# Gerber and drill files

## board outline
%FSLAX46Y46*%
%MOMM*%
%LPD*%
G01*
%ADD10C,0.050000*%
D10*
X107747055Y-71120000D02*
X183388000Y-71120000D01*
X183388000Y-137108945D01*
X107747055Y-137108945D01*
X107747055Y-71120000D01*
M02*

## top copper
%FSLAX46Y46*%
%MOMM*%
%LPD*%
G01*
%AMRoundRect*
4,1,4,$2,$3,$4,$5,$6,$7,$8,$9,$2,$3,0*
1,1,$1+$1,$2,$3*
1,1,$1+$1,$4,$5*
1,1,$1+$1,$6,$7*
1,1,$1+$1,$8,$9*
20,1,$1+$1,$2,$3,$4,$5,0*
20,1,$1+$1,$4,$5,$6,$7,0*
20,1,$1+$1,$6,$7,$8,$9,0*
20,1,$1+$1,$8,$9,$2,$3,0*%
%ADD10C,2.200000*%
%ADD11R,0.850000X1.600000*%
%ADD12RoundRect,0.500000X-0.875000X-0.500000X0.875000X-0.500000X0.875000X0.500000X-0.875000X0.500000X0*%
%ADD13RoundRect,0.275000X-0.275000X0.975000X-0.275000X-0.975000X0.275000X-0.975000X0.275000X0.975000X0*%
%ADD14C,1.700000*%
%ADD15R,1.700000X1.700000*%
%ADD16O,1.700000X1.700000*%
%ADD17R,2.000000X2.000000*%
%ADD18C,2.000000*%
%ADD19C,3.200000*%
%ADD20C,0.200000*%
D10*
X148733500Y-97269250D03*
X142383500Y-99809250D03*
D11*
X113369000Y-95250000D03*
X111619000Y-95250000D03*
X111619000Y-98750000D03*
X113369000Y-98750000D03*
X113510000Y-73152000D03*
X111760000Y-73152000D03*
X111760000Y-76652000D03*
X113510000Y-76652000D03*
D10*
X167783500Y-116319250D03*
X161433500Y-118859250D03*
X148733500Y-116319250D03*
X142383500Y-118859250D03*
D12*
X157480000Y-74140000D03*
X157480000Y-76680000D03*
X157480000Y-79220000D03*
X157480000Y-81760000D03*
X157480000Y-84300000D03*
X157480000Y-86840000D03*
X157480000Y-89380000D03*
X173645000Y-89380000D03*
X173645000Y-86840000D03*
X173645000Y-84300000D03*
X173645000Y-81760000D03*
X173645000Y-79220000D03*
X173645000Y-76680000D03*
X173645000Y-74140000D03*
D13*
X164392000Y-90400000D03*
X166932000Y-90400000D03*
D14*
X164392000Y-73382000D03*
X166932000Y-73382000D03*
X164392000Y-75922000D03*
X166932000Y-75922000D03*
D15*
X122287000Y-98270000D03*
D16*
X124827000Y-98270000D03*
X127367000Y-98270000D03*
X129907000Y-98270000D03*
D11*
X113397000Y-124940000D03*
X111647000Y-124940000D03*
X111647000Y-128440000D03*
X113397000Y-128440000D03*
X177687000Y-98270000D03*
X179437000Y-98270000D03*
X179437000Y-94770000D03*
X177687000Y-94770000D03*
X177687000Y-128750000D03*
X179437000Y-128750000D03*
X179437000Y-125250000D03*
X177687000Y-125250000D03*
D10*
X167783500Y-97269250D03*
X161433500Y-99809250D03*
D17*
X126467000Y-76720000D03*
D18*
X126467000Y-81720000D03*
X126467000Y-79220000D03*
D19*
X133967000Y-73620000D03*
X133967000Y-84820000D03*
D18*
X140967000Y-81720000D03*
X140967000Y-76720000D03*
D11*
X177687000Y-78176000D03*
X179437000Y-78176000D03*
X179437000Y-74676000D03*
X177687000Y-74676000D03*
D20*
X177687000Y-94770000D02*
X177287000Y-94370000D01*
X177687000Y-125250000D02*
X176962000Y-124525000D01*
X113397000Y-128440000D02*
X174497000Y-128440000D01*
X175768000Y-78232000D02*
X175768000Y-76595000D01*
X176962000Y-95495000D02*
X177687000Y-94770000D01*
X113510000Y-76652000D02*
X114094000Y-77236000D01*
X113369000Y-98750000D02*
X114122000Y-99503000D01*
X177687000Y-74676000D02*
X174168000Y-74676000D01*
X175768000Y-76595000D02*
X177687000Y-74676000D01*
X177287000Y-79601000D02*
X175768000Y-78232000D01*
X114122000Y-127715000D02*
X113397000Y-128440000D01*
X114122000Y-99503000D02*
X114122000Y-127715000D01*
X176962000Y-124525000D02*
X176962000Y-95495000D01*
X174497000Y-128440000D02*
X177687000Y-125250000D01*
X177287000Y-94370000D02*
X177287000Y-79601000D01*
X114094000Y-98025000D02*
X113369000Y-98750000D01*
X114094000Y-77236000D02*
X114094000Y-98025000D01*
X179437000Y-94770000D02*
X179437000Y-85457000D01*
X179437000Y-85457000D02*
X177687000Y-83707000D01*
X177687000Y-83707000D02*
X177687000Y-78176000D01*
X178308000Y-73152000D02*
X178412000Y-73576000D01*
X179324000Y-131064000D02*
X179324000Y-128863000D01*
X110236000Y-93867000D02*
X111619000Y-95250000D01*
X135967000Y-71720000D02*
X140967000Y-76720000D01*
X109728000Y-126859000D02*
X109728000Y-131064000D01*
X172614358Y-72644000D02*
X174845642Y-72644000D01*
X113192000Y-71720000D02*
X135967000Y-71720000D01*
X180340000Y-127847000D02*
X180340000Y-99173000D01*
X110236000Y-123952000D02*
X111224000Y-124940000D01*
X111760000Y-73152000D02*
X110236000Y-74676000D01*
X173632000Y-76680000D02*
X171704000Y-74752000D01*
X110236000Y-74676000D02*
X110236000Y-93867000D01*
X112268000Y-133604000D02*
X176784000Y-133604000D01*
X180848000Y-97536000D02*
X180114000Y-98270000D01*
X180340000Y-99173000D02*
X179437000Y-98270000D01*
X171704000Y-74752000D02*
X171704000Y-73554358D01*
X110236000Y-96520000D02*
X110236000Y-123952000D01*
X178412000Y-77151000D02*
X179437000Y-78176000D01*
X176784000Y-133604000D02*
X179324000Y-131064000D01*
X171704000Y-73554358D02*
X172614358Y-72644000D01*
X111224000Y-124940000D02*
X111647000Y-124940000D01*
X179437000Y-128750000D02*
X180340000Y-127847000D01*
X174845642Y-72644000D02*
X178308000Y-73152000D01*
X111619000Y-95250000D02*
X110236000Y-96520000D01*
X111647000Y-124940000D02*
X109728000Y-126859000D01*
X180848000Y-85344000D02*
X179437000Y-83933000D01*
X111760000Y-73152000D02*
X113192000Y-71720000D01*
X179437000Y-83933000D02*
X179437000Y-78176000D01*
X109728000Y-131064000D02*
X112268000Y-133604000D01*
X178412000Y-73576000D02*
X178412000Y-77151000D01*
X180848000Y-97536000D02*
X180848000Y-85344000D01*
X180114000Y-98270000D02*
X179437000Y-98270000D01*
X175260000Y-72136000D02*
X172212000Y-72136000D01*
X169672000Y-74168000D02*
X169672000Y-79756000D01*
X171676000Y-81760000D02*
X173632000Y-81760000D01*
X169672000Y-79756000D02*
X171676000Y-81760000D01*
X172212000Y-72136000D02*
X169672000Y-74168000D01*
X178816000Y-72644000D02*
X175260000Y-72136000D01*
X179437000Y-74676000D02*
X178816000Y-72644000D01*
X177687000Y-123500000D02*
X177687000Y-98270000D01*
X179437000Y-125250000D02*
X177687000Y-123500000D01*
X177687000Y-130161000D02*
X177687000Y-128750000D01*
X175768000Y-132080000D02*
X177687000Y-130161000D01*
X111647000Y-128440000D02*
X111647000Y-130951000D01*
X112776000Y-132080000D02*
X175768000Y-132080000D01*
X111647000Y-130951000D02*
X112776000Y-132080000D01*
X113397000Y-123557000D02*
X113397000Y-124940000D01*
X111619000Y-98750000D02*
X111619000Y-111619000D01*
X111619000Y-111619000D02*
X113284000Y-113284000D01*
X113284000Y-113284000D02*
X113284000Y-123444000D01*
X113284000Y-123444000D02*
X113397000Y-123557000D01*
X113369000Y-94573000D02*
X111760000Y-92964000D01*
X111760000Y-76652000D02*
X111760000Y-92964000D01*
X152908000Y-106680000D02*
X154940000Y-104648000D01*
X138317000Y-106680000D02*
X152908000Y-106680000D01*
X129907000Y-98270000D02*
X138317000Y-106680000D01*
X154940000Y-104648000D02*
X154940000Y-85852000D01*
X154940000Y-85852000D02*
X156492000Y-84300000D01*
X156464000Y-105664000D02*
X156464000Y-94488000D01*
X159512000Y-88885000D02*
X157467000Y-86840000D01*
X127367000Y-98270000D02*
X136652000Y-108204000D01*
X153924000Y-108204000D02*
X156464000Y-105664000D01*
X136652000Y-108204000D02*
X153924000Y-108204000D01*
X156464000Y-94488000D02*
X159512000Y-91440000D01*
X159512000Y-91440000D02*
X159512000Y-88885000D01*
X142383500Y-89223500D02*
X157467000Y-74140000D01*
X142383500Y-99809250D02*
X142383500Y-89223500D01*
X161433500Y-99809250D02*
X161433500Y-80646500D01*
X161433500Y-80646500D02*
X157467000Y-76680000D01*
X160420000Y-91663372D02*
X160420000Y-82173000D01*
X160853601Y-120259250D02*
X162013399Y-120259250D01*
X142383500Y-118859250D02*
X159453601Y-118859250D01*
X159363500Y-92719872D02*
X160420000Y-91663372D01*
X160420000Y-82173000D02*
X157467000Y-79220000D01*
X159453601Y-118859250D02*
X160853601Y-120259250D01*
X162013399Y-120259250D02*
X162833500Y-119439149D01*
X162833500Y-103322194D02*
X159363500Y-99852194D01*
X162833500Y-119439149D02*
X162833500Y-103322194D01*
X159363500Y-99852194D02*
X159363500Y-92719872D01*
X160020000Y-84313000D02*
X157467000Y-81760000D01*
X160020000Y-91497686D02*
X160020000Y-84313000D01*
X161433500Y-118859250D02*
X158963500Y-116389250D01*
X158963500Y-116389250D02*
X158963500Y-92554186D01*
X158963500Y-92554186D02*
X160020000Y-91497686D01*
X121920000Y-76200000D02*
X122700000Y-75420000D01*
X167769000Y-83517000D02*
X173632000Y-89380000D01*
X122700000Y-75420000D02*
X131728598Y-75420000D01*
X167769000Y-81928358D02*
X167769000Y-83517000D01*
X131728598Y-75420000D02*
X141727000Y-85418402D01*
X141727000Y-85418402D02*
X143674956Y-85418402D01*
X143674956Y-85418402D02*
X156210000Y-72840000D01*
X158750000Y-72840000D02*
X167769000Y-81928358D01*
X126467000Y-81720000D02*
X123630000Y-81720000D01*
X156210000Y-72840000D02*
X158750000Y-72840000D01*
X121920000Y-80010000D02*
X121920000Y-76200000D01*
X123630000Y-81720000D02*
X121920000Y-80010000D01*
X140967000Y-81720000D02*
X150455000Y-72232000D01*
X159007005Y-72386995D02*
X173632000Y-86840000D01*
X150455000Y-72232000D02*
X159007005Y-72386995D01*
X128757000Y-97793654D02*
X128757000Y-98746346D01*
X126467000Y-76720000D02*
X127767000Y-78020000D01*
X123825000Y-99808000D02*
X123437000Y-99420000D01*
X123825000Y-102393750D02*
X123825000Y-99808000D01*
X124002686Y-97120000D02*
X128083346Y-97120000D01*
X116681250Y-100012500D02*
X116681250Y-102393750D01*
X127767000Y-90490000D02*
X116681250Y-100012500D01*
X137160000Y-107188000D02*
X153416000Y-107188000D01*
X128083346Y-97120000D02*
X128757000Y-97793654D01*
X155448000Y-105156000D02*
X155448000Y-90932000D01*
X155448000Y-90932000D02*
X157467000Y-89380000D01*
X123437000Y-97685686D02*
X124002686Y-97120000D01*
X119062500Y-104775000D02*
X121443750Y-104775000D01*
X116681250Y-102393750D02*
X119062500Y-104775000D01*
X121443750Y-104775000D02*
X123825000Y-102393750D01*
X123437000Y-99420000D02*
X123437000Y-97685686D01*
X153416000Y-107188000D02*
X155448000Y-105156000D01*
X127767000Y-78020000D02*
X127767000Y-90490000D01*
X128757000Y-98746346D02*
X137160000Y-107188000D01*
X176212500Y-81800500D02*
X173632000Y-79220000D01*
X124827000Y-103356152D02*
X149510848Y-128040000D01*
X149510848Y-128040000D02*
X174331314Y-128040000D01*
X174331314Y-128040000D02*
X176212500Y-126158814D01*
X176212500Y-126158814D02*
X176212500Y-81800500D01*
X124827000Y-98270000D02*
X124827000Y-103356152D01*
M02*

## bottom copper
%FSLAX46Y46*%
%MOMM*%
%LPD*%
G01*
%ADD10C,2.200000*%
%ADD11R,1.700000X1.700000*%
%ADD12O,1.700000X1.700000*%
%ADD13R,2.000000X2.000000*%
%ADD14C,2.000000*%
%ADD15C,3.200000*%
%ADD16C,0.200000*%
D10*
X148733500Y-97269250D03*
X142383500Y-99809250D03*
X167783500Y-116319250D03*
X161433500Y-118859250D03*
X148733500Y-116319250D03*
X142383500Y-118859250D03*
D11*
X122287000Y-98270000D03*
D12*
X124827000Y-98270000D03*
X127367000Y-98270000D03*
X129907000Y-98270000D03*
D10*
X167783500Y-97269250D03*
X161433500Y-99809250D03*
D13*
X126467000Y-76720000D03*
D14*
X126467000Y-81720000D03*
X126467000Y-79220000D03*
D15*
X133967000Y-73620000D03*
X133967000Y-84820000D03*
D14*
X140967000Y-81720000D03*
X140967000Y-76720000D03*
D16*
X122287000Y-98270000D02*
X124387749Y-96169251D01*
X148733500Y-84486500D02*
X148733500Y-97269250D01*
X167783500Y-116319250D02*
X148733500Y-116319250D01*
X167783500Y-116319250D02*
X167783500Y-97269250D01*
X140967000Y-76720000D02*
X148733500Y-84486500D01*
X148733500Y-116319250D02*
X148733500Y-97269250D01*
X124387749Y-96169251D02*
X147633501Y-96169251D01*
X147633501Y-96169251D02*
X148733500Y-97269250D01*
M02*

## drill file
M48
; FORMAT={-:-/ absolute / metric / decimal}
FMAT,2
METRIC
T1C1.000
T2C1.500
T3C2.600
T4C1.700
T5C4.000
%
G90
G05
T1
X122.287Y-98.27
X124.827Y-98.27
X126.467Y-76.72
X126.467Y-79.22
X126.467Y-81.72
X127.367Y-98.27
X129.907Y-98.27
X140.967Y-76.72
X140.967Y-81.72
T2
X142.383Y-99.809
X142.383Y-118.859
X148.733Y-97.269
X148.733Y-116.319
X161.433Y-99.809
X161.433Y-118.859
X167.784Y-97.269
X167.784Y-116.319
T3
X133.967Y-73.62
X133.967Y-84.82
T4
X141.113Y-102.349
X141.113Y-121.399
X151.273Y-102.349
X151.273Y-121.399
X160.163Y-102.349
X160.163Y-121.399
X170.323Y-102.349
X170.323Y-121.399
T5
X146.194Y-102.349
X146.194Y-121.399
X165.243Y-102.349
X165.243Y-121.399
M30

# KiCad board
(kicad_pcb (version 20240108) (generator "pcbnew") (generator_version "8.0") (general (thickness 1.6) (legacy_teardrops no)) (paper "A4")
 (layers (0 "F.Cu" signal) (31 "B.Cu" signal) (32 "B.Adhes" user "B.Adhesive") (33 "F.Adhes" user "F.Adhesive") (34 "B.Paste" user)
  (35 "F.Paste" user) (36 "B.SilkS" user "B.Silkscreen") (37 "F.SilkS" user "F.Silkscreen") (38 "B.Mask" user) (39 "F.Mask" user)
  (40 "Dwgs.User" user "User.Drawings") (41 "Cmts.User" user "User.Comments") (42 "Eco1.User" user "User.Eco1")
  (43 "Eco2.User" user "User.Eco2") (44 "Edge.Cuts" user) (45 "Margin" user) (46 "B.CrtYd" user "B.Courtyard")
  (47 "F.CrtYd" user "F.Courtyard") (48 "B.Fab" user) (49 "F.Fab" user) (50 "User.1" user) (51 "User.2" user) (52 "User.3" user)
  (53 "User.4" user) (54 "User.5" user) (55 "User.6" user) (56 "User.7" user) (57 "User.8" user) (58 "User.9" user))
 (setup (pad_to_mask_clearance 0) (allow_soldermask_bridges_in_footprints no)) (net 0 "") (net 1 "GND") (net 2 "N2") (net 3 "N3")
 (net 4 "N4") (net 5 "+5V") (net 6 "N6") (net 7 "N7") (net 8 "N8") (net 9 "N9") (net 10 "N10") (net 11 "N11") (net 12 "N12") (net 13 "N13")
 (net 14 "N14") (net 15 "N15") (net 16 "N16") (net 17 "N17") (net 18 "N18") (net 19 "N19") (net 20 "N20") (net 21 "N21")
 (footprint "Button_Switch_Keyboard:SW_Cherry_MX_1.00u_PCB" (layer "F.Cu") (at 148.7335 97.26925)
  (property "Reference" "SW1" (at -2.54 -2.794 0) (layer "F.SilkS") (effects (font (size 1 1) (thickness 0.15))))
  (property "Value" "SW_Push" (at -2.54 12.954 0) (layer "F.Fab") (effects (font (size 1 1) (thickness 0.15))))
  (pad "" np_thru_hole circle (at -7.62 5.08) (size 1.7 1.7) (drill 1.7) (layers "*.Cu" "*.Mask"))
  (pad "" np_thru_hole circle (at -2.54 5.08) (size 4 4) (drill 4) (layers "*.Cu" "*.Mask"))
  (pad "" np_thru_hole circle (at 2.54 5.08) (size 1.7 1.7) (drill 1.7) (layers "*.Cu" "*.Mask"))
  (pad "1" thru_hole circle (at 0 0) (size 2.2 2.2) (drill 1.5) (layers "*.Cu" "*.Mask") (remove_unused_layers no) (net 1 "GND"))
  (pad "2" thru_hole circle (at -6.35 2.54) (size 2.2 2.2) (drill 1.5) (layers "*.Cu" "*.Mask") (remove_unused_layers no) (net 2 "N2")))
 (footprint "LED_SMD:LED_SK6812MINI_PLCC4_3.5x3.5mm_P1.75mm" (layer "F.Cu") (at 112.494 97 -90)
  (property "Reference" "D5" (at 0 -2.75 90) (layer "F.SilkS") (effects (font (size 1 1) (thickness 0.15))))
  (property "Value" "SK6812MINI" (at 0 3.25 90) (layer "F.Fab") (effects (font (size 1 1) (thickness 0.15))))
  (pad "1" smd rect (at -1.75 -0.875 270) (size 1.6 0.85) (layers "F.Cu" "F.Paste" "F.Mask") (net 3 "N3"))
  (pad "2" smd rect (at -1.75 0.875 270) (size 1.6 0.85) (layers "F.Cu" "F.Paste" "F.Mask") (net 1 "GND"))
  (pad "3" smd rect (at 1.75 0.875 270) (size 1.6 0.85) (layers "F.Cu" "F.Paste" "F.Mask") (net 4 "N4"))
  (pad "4" smd rect (at 1.75 -0.875 270) (size 1.6 0.85) (layers "F.Cu" "F.Paste" "F.Mask") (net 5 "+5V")))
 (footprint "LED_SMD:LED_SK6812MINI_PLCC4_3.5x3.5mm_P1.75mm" (layer "F.Cu") (at 112.635 74.902 -90)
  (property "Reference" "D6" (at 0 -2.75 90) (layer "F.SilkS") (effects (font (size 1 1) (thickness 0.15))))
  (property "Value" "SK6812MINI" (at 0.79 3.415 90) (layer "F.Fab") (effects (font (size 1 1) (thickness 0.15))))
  (pad "1" smd rect (at -1.75 -0.875 270) (size 1.6 0.85) (layers "F.Cu" "F.Paste" "F.Mask") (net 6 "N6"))
  (pad "2" smd rect (at -1.75 0.875 270) (size 1.6 0.85) (layers "F.Cu" "F.Paste" "F.Mask") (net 1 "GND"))
  (pad "3" smd rect (at 1.75 0.875 270) (size 1.6 0.85) (layers "F.Cu" "F.Paste" "F.Mask") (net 3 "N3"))
  (pad "4" smd rect (at 1.75 -0.875 270) (size 1.6 0.85) (layers "F.Cu" "F.Paste" "F.Mask") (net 5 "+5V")))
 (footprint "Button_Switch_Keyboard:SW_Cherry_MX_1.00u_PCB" (layer "F.Cu") (at 167.7835 116.31925)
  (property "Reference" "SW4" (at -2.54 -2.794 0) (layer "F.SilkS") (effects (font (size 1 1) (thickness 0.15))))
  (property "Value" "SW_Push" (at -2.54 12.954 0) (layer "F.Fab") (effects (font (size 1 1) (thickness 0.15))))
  (pad "" np_thru_hole circle (at -7.62 5.08) (size 1.7 1.7) (drill 1.7) (layers "*.Cu" "*.Mask"))
  (pad "" np_thru_hole circle (at -2.54 5.08) (size 4 4) (drill 4) (layers "F&B.Cu" "*.Mask"))
  (pad "" np_thru_hole circle (at 2.54 5.08) (size 1.7 1.7) (drill 1.7) (layers "*.Cu" "*.Mask"))
  (pad "1" thru_hole circle (at 0 0) (size 2.2 2.2) (drill 1.5) (layers "*.Cu" "*.Mask") (remove_unused_layers no) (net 1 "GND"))
  (pad "2" thru_hole circle (at -6.35 2.54) (size 2.2 2.2) (drill 1.5) (layers "*.Cu" "*.Mask") (remove_unused_layers no) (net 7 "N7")))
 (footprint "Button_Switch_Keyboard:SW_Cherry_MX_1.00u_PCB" (layer "F.Cu") (at 148.7335 116.31925)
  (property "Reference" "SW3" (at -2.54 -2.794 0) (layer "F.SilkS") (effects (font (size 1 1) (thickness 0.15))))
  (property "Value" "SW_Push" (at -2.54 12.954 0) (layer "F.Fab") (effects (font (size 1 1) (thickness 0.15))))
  (pad "" np_thru_hole circle (at -7.62 5.08) (size 1.7 1.7) (drill 1.7) (layers "*.Cu" "*.Mask"))
  (pad "" np_thru_hole circle (at -2.54 5.08) (size 4 4) (drill 4) (layers "F&B.Cu" "*.Mask"))
  (pad "" np_thru_hole circle (at 2.54 5.08) (size 1.7 1.7) (drill 1.7) (layers "*.Cu" "*.Mask"))
  (pad "1" thru_hole circle (at 0 0) (size 2.2 2.2) (drill 1.5) (layers "*.Cu" "*.Mask") (remove_unused_layers no) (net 1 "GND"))
  (pad "2" thru_hole circle (at -6.35 2.54) (size 2.2 2.2) (drill 1.5) (layers "*.Cu" "*.Mask") (remove_unused_layers no) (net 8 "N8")))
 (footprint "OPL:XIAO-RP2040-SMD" (layer "F.Cu") (at 165.48 81.76)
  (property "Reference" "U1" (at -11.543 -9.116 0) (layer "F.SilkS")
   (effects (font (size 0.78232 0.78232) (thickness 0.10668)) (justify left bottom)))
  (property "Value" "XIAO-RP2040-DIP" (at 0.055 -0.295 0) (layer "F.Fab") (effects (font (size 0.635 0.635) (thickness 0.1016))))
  (pad "1" smd roundrect (at -8 -7.62) (size 2.75 2) (layers "F.Cu" "F.Paste" "F.Mask") (roundrect_rratio 0.25) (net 2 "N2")
   (solder_mask_margin 0.0508) (thermal_bridge_angle 45))
  (pad "2" smd roundrect (at -8 -5.08) (size 2.75 2) (layers "F.Cu" "F.Paste" "F.Mask") (roundrect_rratio 0.25) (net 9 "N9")
   (solder_mask_margin 0.0508) (thermal_bridge_angle 45))
  (pad "3" smd roundrect (at -8 -2.54) (size 2.75 2) (layers "F.Cu" "F.Paste" "F.Mask") (roundrect_rratio 0.25) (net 8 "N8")
   (solder_mask_margin 0.0508) (thermal_bridge_angle 45))
  (pad "4" smd roundrect (at -8 0) (size 2.75 2) (layers "F.Cu" "F.Paste" "F.Mask") (roundrect_rratio 0.25) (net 7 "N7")
   (solder_mask_margin 0.0508) (thermal_bridge_angle 45))
  (pad "5" smd roundrect (at -8 2.54) (size 2.75 2) (layers "F.Cu" "F.Paste" "F.Mask") (roundrect_rratio 0.25) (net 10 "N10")
   (solder_mask_margin 0.0508) (thermal_bridge_angle 45))
  (pad "6" smd roundrect (at -8 5.08) (size 2.75 2) (layers "F.Cu" "F.Paste" "F.Mask") (roundrect_rratio 0.25) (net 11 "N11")
   (solder_mask_margin 0.0508) (thermal_bridge_angle 45))
  (pad "7" smd roundrect (at -8 7.62) (size 2.75 2) (layers "F.Cu" "F.Paste" "F.Mask") (roundrect_rratio 0.25) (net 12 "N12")
   (solder_mask_margin 0.0508) (thermal_bridge_angle 45))
  (pad "8" smd roundrect (at 8.165 7.62) (size 2.75 2) (layers "F.Cu" "F.Paste" "F.Mask") (roundrect_rratio 0.25) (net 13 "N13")
   (solder_mask_margin 0.0508) (thermal_bridge_angle 45))
  (pad "9" smd roundrect (at 8.165 5.08) (size 2.75 2) (layers "F.Cu" "F.Paste" "F.Mask") (roundrect_rratio 0.25) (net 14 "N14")
   (solder_mask_margin 0.0508) (thermal_bridge_angle 45))
  (pad "10" smd roundrect (at 8.165 2.54) (size 2.75 2) (layers "F.Cu" "F.Paste" "F.Mask") (roundrect_rratio 0.25) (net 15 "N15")
   (solder_mask_margin 0.0508) (thermal_bridge_angle 45))
  (pad "11" smd roundrect (at 8.165 0) (size 2.75 2) (layers "F.Cu" "F.Paste" "F.Mask") (roundrect_rratio 0.25) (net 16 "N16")
   (solder_mask_margin 0.0508) (thermal_bridge_angle 45))
  (pad "12" smd roundrect (at 8.165 -2.54) (size 2.75 2) (layers "F.Cu" "F.Paste" "F.Mask") (roundrect_rratio 0.25) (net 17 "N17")
   (solder_mask_margin 0.0508) (thermal_bridge_angle 45))
  (pad "13" smd roundrect (at 8.165 -5.08) (size 2.75 2) (layers "F.Cu" "F.Paste" "F.Mask") (roundrect_rratio 0.25) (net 1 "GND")
   (solder_mask_margin 0.0508) (thermal_bridge_angle 45))
  (pad "14" smd roundrect (at 8.165 -7.62) (size 2.75 2) (layers "F.Cu" "F.Paste" "F.Mask") (roundrect_rratio 0.25) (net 5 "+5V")
   (solder_mask_margin 0.0508) (thermal_bridge_angle 45))
  (pad "15" smd roundrect (at -1.088 8.64 270) (size 2.5 1.1) (layers "F.Cu" "F.Paste" "F.Mask") (roundrect_rratio 0.25)
   (thermal_bridge_angle 45))
  (pad "16" smd roundrect (at 1.452 8.64 270) (size 2.5 1.1) (layers "F.Cu" "F.Paste" "F.Mask") (roundrect_rratio 0.25)
   (thermal_bridge_angle 45))
  (pad "17" smd circle (at -1.088 -8.378) (size 1.7 1.7) (layers "F.Cu" "F.Paste" "F.Mask"))
  (pad "18" smd circle (at 1.452 -8.378) (size 1.7 1.7) (layers "F.Cu" "F.Paste" "F.Mask"))
  (pad "19" smd circle (at -1.088 -5.838) (size 1.7 1.7) (layers "F.Cu" "F.Paste" "F.Mask"))
  (pad "20" smd circle (at 1.452 -5.838) (size 1.7 1.7) (layers "F.Cu" "F.Paste" "F.Mask")))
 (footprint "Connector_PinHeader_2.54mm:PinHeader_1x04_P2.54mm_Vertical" (layer "F.Cu") (at 122.287 98.27 90)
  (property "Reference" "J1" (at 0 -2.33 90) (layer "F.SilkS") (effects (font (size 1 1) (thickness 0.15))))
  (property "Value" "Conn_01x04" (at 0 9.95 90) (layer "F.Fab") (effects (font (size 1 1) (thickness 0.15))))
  (pad "1" thru_hole rect (at 0 0 90) (size 1.7 1.7) (drill 1) (layers "*.Cu" "*.Mask") (remove_unused_layers no) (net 1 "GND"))
  (pad "2" thru_hole oval (at 0 2.54 90) (size 1.7 1.7) (drill 1) (layers "*.Cu" "*.Mask") (remove_unused_layers no) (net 17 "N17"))
  (pad "3" thru_hole oval (at 0 5.08 90) (size 1.7 1.7) (drill 1) (layers "*.Cu" "*.Mask") (remove_unused_layers no) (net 11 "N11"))
  (pad "4" thru_hole oval (at 0 7.62 90) (size 1.7 1.7) (drill 1) (layers "*.Cu" "*.Mask") (remove_unused_layers no) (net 10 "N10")))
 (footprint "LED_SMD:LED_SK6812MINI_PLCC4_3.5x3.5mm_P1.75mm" (layer "F.Cu") (at 112.522 126.69 -90)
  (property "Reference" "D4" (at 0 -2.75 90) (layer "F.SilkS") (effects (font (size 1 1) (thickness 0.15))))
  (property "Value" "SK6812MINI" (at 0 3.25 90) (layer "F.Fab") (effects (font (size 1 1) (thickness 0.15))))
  (pad "1" smd rect (at -1.75 -0.875 270) (size 1.6 0.85) (layers "F.Cu" "F.Paste" "F.Mask") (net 4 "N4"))
  (pad "2" smd rect (at -1.75 0.875 270) (size 1.6 0.85) (layers "F.Cu" "F.Paste" "F.Mask") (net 1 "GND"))
  (pad "3" smd rect (at 1.75 0.875 270) (size 1.6 0.85) (layers "F.Cu" "F.Paste" "F.Mask") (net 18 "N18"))
  (pad "4" smd rect (at 1.75 -0.875 270) (size 1.6 0.85) (layers "F.Cu" "F.Paste" "F.Mask") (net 5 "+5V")))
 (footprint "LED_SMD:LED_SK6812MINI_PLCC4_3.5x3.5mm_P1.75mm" (layer "F.Cu") (at 178.562 96.52 90)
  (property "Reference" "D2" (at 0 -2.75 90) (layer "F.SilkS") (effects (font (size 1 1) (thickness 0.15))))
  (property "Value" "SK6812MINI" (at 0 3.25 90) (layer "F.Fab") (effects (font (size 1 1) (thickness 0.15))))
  (pad "1" smd rect (at -1.75 -0.875 90) (size 1.6 0.85) (layers "F.Cu" "F.Paste" "F.Mask") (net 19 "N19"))
  (pad "2" smd rect (at -1.75 0.875 90) (size 1.6 0.85) (layers "F.Cu" "F.Paste" "F.Mask") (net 1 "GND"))
  (pad "3" smd rect (at 1.75 0.875 90) (size 1.6 0.85) (layers "F.Cu" "F.Paste" "F.Mask") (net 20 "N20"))
  (pad "4" smd rect (at 1.75 -0.875 90) (size 1.6 0.85) (layers "F.Cu" "F.Paste" "F.Mask") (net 5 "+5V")))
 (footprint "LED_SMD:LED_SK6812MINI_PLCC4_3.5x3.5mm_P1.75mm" (layer "F.Cu") (at 178.562 127 90)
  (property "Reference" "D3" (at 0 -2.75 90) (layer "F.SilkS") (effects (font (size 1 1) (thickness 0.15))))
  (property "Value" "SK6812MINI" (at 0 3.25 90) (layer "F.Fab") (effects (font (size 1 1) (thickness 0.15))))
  (pad "1" smd rect (at -1.75 -0.875 90) (size 1.6 0.85) (layers "F.Cu" "F.Paste" "F.Mask") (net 18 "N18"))
  (pad "2" smd rect (at -1.75 0.875 90) (size 1.6 0.85) (layers "F.Cu" "F.Paste" "F.Mask") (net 1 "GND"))
  (pad "3" smd rect (at 1.75 0.875 90) (size 1.6 0.85) (layers "F.Cu" "F.Paste" "F.Mask") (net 19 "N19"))
  (pad "4" smd rect (at 1.75 -0.875 90) (size 1.6 0.85) (layers "F.Cu" "F.Paste" "F.Mask") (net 5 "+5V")))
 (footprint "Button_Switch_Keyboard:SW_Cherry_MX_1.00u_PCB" (layer "F.Cu") (at 167.7835 97.26925)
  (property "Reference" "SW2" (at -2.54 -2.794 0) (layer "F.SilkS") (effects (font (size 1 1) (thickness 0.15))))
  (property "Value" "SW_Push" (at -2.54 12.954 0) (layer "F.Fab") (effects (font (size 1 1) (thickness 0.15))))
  (pad "" np_thru_hole circle (at -7.62 5.08) (size 1.7 1.7) (drill 1.7) (layers "*.Cu" "*.Mask"))
  (pad "" np_thru_hole circle (at -2.54 5.08) (size 4 4) (drill 4) (layers "F&B.Cu" "*.Mask"))
  (pad "" np_thru_hole circle (at 2.54 5.08) (size 1.7 1.7) (drill 1.7) (layers "*.Cu" "*.Mask"))
  (pad "1" thru_hole circle (at 0 0) (size 2.2 2.2) (drill 1.5) (layers "*.Cu" "*.Mask") (remove_unused_layers no) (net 1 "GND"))
  (pad "2" thru_hole circle (at -6.35 2.54) (size 2.2 2.2) (drill 1.5) (layers "*.Cu" "*.Mask") (remove_unused_layers no) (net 9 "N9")))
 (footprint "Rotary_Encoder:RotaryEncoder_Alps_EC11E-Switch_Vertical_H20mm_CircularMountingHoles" (layer "F.Cu") (at 126.467 76.72)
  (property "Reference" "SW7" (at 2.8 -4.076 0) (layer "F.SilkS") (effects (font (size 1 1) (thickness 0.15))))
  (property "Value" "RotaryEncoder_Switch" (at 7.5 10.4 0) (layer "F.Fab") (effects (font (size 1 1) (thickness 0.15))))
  (pad "A" thru_hole rect (at 0 0) (size 2 2) (drill 1) (layers "*.Cu" "*.Mask") (remove_unused_layers no) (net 12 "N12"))
  (pad "B" thru_hole circle (at 0 5) (size 2 2) (drill 1) (layers "*.Cu" "*.Mask") (remove_unused_layers no) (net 13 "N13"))
  (pad "C" thru_hole circle (at 0 2.5) (size 2 2) (drill 1) (layers "*.Cu" "*.Mask") (remove_unused_layers no) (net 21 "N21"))
  (pad "MP" thru_hole circle (at 7.5 -3.1) (size 3.2 3.2) (drill 2.6) (layers "*.Cu" "*.Mask") (remove_unused_layers no))
  (pad "MP" thru_hole circle (at 7.5 8.1) (size 3.2 3.2) (drill 2.6) (layers "*.Cu" "*.Mask") (remove_unused_layers no))
  (pad "S1" thru_hole circle (at 14.5 5) (size 2 2) (drill 1) (layers "*.Cu" "*.Mask") (remove_unused_layers no) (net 14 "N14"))
  (pad "S2" thru_hole circle (at 14.5 0) (size 2 2) (drill 1) (layers "*.Cu" "*.Mask") (remove_unused_layers no) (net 1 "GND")))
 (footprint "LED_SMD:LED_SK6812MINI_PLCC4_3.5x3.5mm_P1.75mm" (layer "F.Cu") (at 178.562 76.426 90)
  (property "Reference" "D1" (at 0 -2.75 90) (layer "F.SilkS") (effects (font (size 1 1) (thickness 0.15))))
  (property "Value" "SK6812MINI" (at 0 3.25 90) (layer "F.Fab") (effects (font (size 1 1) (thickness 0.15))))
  (pad "1" smd rect (at -1.75 -0.875 90) (size 1.6 0.85) (layers "F.Cu" "F.Paste" "F.Mask") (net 20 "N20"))
  (pad "2" smd rect (at -1.75 0.875 90) (size 1.6 0.85) (layers "F.Cu" "F.Paste" "F.Mask") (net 1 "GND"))
  (pad "3" smd rect (at 1.75 0.875 90) (size 1.6 0.85) (layers "F.Cu" "F.Paste" "F.Mask") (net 16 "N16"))
  (pad "4" smd rect (at 1.75 -0.875 90) (size 1.6 0.85) (layers "F.Cu" "F.Paste" "F.Mask") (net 5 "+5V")))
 (gr_rect (start 107.747055 71.12) (end 183.388 137.108945) (stroke (width 0.05) (type default)) (fill none) (layer "Edge.Cuts"))
 (segment (start 177.687 94.77) (end 177.287 94.37) (width 0.2) (layer "F.Cu") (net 5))
 (segment (start 177.687 125.25) (end 176.962 124.525) (width 0.2) (layer "F.Cu") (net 5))
 (segment (start 113.397 128.44) (end 174.497 128.44) (width 0.2) (layer "F.Cu") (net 5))
 (segment (start 175.768 78.232) (end 175.768 76.595) (width 0.2) (layer "F.Cu") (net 5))
 (segment (start 176.962 95.495) (end 177.687 94.77) (width 0.2) (layer "F.Cu") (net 5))
 (segment (start 113.51 76.652) (end 114.094 77.236) (width 0.2) (layer "F.Cu") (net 5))
 (segment (start 113.369 98.75) (end 114.122 99.503) (width 0.2) (layer "F.Cu") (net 5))
 (segment (start 177.687 74.676) (end 174.168 74.676) (width 0.2) (layer "F.Cu") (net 5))
 (segment (start 175.768 76.595) (end 177.687 74.676) (width 0.2) (layer "F.Cu") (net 5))
 (segment (start 177.287 79.601) (end 175.768 78.232) (width 0.2) (layer "F.Cu") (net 5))
 (segment (start 114.122 127.715) (end 113.397 128.44) (width 0.2) (layer "F.Cu") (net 5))
 (segment (start 114.122 99.503) (end 114.122 127.715) (width 0.2) (layer "F.Cu") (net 5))
 (segment (start 176.962 124.525) (end 176.962 95.495) (width 0.2) (layer "F.Cu") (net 5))
 (segment (start 174.497 128.44) (end 177.687 125.25) (width 0.2) (layer "F.Cu") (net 5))
 (segment (start 177.287 94.37) (end 177.287 79.601) (width 0.2) (layer "F.Cu") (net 5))
 (segment (start 114.094 98.025) (end 113.369 98.75) (width 0.2) (layer "F.Cu") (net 5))
 (segment (start 114.094 77.236) (end 114.094 98.025) (width 0.2) (layer "F.Cu") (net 5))
 (segment (start 179.437 94.77) (end 179.437 85.457) (width 0.2) (layer "F.Cu") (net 20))
 (segment (start 179.437 85.457) (end 177.687 83.707) (width 0.2) (layer "F.Cu") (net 20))
 (segment (start 177.687 83.707) (end 177.687 78.176) (width 0.2) (layer "F.Cu") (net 20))
 (segment (start 178.308 73.152) (end 178.412 73.576) (width 0.2) (layer "F.Cu") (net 1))
 (segment (start 179.324 131.064) (end 179.324 128.863) (width 0.2) (layer "F.Cu") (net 1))
 (segment (start 110.236 93.867) (end 111.619 95.25) (width 0.2) (layer "F.Cu") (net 1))
 (segment (start 135.967 71.72) (end 140.967 76.72) (width 0.2) (layer "F.Cu") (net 1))
 (segment (start 109.728 126.859) (end 109.728 131.064) (width 0.2) (layer "F.Cu") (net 1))
 (segment (start 172.614358 72.644) (end 174.845642 72.644) (width 0.2) (layer "F.Cu") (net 1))
 (segment (start 113.192 71.72) (end 135.967 71.72) (width 0.2) (layer "F.Cu") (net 1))
 (segment (start 180.34 127.847) (end 180.34 99.173) (width 0.2) (layer "F.Cu") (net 1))
 (segment (start 110.236 123.952) (end 111.224 124.94) (width 0.2) (layer "F.Cu") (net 1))
 (segment (start 111.76 73.152) (end 110.236 74.676) (width 0.2) (layer "F.Cu") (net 1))
 (segment (start 173.632 76.68) (end 171.704 74.752) (width 0.2) (layer "F.Cu") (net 1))
 (segment (start 110.236 74.676) (end 110.236 93.867) (width 0.2) (layer "F.Cu") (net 1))
 (segment (start 112.268 133.604) (end 176.784 133.604) (width 0.2) (layer "F.Cu") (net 1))
 (segment (start 180.848 97.536) (end 180.114 98.27) (width 0.2) (layer "F.Cu") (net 1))
 (segment (start 180.34 99.173) (end 179.437 98.27) (width 0.2) (layer "F.Cu") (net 1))
 (segment (start 171.704 74.752) (end 171.704 73.554358) (width 0.2) (layer "F.Cu") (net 1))
 (segment (start 110.236 96.52) (end 110.236 123.952) (width 0.2) (layer "F.Cu") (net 1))
 (segment (start 178.412 77.151) (end 179.437 78.176) (width 0.2) (layer "F.Cu") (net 1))
 (segment (start 176.784 133.604) (end 179.324 131.064) (width 0.2) (layer "F.Cu") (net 1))
 (segment (start 171.704 73.554358) (end 172.614358 72.644) (width 0.2) (layer "F.Cu") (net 1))
 (segment (start 111.224 124.94) (end 111.647 124.94) (width 0.2) (layer "F.Cu") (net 1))
 (segment (start 179.437 128.75) (end 180.34 127.847) (width 0.2) (layer "F.Cu") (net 1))
 (segment (start 174.845642 72.644) (end 178.308 73.152) (width 0.2) (layer "F.Cu") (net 1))
 (segment (start 111.619 95.25) (end 110.236 96.52) (width 0.2) (layer "F.Cu") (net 1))
 (segment (start 111.647 124.94) (end 109.728 126.859) (width 0.2) (layer "F.Cu") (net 1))
 (segment (start 180.848 85.344) (end 179.437 83.933) (width 0.2) (layer "F.Cu") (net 1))
 (segment (start 111.76 73.152) (end 113.192 71.72) (width 0.2) (layer "F.Cu") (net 1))
 (segment (start 179.437 83.933) (end 179.437 78.176) (width 0.2) (layer "F.Cu") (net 1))
 (segment (start 109.728 131.064) (end 112.268 133.604) (width 0.2) (layer "F.Cu") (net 1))
 (segment (start 178.412 73.576) (end 178.412 77.151) (width 0.2) (layer "F.Cu") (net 1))
 (segment (start 180.848 97.536) (end 180.848 85.344) (width 0.2) (layer "F.Cu") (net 1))
 (segment (start 180.114 98.27) (end 179.437 98.27) (width 0.2) (layer "F.Cu") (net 1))
 (segment (start 122.287 98.27) (end 124.387749 96.169251) (width 0.2) (layer "B.Cu") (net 1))
 (segment (start 148.7335 84.4865) (end 148.7335 97.26925) (width 0.2) (layer "B.Cu") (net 1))
 (segment (start 167.7835 116.31925) (end 148.7335 116.31925) (width 0.2) (layer "B.Cu") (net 1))
 (segment (start 167.7835 116.31925) (end 167.7835 97.26925) (width 0.2) (layer "B.Cu") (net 1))
 (segment (start 140.967 76.72) (end 148.7335 84.4865) (width 0.2) (layer "B.Cu") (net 1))
 (segment (start 148.7335 116.31925) (end 148.7335 97.26925) (width 0.2) (layer "B.Cu") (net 1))
 (segment (start 124.387749 96.169251) (end 147.633501 96.169251) (width 0.2) (layer "B.Cu") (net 1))
 (segment (start 147.633501 96.169251) (end 148.7335 97.26925) (width 0.2) (layer "B.Cu") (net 1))
 (segment (start 175.26 72.136) (end 172.212 72.136) (width 0.2) (layer "F.Cu") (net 16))
 (segment (start 169.672 74.168) (end 169.672 79.756) (width 0.2) (layer "F.Cu") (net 16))
 (segment (start 171.676 81.76) (end 173.632 81.76) (width 0.2) (layer "F.Cu") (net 16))
 (segment (start 169.672 79.756) (end 171.676 81.76) (width 0.2) (layer "F.Cu") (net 16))
 (segment (start 172.212 72.136) (end 169.672 74.168) (width 0.2) (layer "F.Cu") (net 16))
 (segment (start 178.816 72.644) (end 175.26 72.136) (width 0.2) (layer "F.Cu") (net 16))
 (segment (start 179.437 74.676) (end 178.816 72.644) (width 0.2) (layer "F.Cu") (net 16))
 (segment (start 177.687 123.5) (end 177.687 98.27) (width 0.2) (layer "F.Cu") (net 19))
 (segment (start 179.437 125.25) (end 177.687 123.5) (width 0.2) (layer "F.Cu") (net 19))
 (segment (start 177.687 130.161) (end 177.687 128.75) (width 0.2) (layer "F.Cu") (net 18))
 (segment (start 175.768 132.08) (end 177.687 130.161) (width 0.2) (layer "F.Cu") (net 18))
 (segment (start 111.647 128.44) (end 111.647 130.951) (width 0.2) (layer "F.Cu") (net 18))
 (segment (start 112.776 132.08) (end 175.768 132.08) (width 0.2) (layer "F.Cu") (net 18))
 (segment (start 111.647 130.951) (end 112.776 132.08) (width 0.2) (layer "F.Cu") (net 18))
 (segment (start 113.397 123.557) (end 113.397 124.94) (width 0.2) (layer "F.Cu") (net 4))
 (segment (start 111.619 98.75) (end 111.619 111.619) (width 0.2) (layer "F.Cu") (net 4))
 (segment (start 111.619 111.619) (end 113.284 113.284) (width 0.2) (layer "F.Cu") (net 4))
 (segment (start 113.284 113.284) (end 113.284 123.444) (width 0.2) (layer "F.Cu") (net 4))
 (segment (start 113.284 123.444) (end 113.397 123.557) (width 0.2) (layer "F.Cu") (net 4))
 (segment (start 113.369 94.573) (end 111.76 92.964) (width 0.2) (layer "F.Cu") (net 3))
 (segment (start 111.76 76.652) (end 111.76 92.964) (width 0.2) (layer "F.Cu") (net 3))
 (segment (start 152.908 106.68) (end 154.94 104.648) (width 0.2) (layer "F.Cu") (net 10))
 (segment (start 138.317 106.68) (end 152.908 106.68) (width 0.2) (layer "F.Cu") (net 10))
 (segment (start 129.907 98.27) (end 138.317 106.68) (width 0.2) (layer "F.Cu") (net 10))
 (segment (start 154.94 104.648) (end 154.94 85.852) (width 0.2) (layer "F.Cu") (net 10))
 (segment (start 154.94 85.852) (end 156.492 84.3) (width 0.2) (layer "F.Cu") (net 10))
 (segment (start 156.464 105.664) (end 156.464 94.488) (width 0.2) (layer "F.Cu") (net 11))
 (segment (start 159.512 88.885) (end 157.467 86.84) (width 0.2) (layer "F.Cu") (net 11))
 (segment (start 127.367 98.27) (end 136.652 108.204) (width 0.2) (layer "F.Cu") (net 11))
 (segment (start 153.924 108.204) (end 156.464 105.664) (width 0.2) (layer "F.Cu") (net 11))
 (segment (start 136.652 108.204) (end 153.924 108.204) (width 0.2) (layer "F.Cu") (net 11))
 (segment (start 156.464 94.488) (end 159.512 91.44) (width 0.2) (layer "F.Cu") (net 11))
 (segment (start 159.512 91.44) (end 159.512 88.885) (width 0.2) (layer "F.Cu") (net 11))
 (segment (start 142.3835 89.2235) (end 157.467 74.14) (width 0.2) (layer "F.Cu") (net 2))
 (segment (start 142.3835 99.80925) (end 142.3835 89.2235) (width 0.2) (layer "F.Cu") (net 2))
 (segment (start 161.4335 99.80925) (end 161.4335 80.6465) (width 0.2) (layer "F.Cu") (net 9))
 (segment (start 161.4335 80.6465) (end 157.467 76.68) (width 0.2) (layer "F.Cu") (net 9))
 (segment (start 160.42 91.663372) (end 160.42 82.173) (width 0.2) (layer "F.Cu") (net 8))
 (segment (start 160.853601 120.25925) (end 162.013399 120.25925) (width 0.2) (layer "F.Cu") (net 8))
 (segment (start 142.3835 118.85925) (end 159.453601 118.85925) (width 0.2) (layer "F.Cu") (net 8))
 (segment (start 159.3635 92.719872) (end 160.42 91.663372) (width 0.2) (layer "F.Cu") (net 8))
 (segment (start 160.42 82.173) (end 157.467 79.22) (width 0.2) (layer "F.Cu") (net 8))
 (segment (start 159.453601 118.85925) (end 160.853601 120.25925) (width 0.2) (layer "F.Cu") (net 8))
 (segment (start 162.013399 120.25925) (end 162.8335 119.439149) (width 0.2) (layer "F.Cu") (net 8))
 (segment (start 162.8335 103.322194) (end 159.3635 99.852194) (width 0.2) (layer "F.Cu") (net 8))
 (segment (start 162.8335 119.439149) (end 162.8335 103.322194) (width 0.2) (layer "F.Cu") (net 8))
 (segment (start 159.3635 99.852194) (end 159.3635 92.719872) (width 0.2) (layer "F.Cu") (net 8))
 (segment (start 160.02 84.313) (end 157.467 81.76) (width 0.2) (layer "F.Cu") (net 7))
 (segment (start 160.02 91.497686) (end 160.02 84.313) (width 0.2) (layer "F.Cu") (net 7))
 (segment (start 161.4335 118.85925) (end 158.9635 116.38925) (width 0.2) (layer "F.Cu") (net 7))
 (segment (start 158.9635 116.38925) (end 158.9635 92.554186) (width 0.2) (layer "F.Cu") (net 7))
 (segment (start 158.9635 92.554186) (end 160.02 91.497686) (width 0.2) (layer "F.Cu") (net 7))
 (segment (start 121.92 76.2) (end 122.7 75.42) (width 0.2) (layer "F.Cu") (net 13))
 (segment (start 167.769 83.517) (end 173.632 89.38) (width 0.2) (layer "F.Cu") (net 13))
 (segment (start 122.7 75.42) (end 131.728598 75.42) (width 0.2) (layer "F.Cu") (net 13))
 (segment (start 167.769 81.928358) (end 167.769 83.517) (width 0.2) (layer "F.Cu") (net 13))
 (segment (start 131.728598 75.42) (end 141.727 85.418402) (width 0.2) (layer "F.Cu") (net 13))
 (segment (start 141.727 85.418402) (end 143.674956 85.418402) (width 0.2) (layer "F.Cu") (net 13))
 (segment (start 143.674956 85.418402) (end 156.21 72.84) (width 0.2) (layer "F.Cu") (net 13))
 (segment (start 158.75 72.84) (end 167.769 81.928358) (width 0.2) (layer "F.Cu") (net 13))
 (segment (start 126.467 81.72) (end 123.63 81.72) (width 0.2) (layer "F.Cu") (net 13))
 (segment (start 156.21 72.84) (end 158.75 72.84) (width 0.2) (layer "F.Cu") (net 13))
 (segment (start 121.92 80.01) (end 121.92 76.2) (width 0.2) (layer "F.Cu") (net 13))
 (segment (start 123.63 81.72) (end 121.92 80.01) (width 0.2) (layer "F.Cu") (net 13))
 (segment (start 140.967 81.72) (end 150.455 72.232) (width 0.2) (layer "F.Cu") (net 14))
 (segment (start 159.007005 72.386995) (end 173.632 86.84) (width 0.2) (layer "F.Cu") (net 14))
 (segment (start 150.455 72.232) (end 159.007005 72.386995) (width 0.2) (layer "F.Cu") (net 14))
 (segment (start 128.757 97.793654) (end 128.757 98.746346) (width 0.2) (layer "F.Cu") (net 12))
 (segment (start 126.467 76.72) (end 127.767 78.02) (width 0.2) (layer "F.Cu") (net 12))
 (segment (start 123.825 99.808) (end 123.437 99.42) (width 0.2) (layer "F.Cu") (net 12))
 (segment (start 123.825 102.39375) (end 123.825 99.808) (width 0.2) (layer "F.Cu") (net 12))
 (segment (start 124.002686 97.12) (end 128.083346 97.12) (width 0.2) (layer "F.Cu") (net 12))
 (segment (start 116.68125 100.0125) (end 116.68125 102.39375) (width 0.2) (layer "F.Cu") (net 12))
 (segment (start 127.767 90.49) (end 116.68125 100.0125) (width 0.2) (layer "F.Cu") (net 12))
 (segment (start 137.16 107.188) (end 153.416 107.188) (width 0.2) (layer "F.Cu") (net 12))
 (segment (start 128.083346 97.12) (end 128.757 97.793654) (width 0.2) (layer "F.Cu") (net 12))
 (segment (start 155.448 105.156) (end 155.448 90.932) (width 0.2) (layer "F.Cu") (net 12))
 (segment (start 155.448 90.932) (end 157.467 89.38) (width 0.2) (layer "F.Cu") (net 12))
 (segment (start 123.437 97.685686) (end 124.002686 97.12) (width 0.2) (layer "F.Cu") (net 12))
 (segment (start 119.0625 104.775) (end 121.44375 104.775) (width 0.2) (layer "F.Cu") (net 12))
 (segment (start 116.68125 102.39375) (end 119.0625 104.775) (width 0.2) (layer "F.Cu") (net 12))
 (segment (start 121.44375 104.775) (end 123.825 102.39375) (width 0.2) (layer "F.Cu") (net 12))
 (segment (start 123.437 99.42) (end 123.437 97.685686) (width 0.2) (layer "F.Cu") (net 12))
 (segment (start 153.416 107.188) (end 155.448 105.156) (width 0.2) (layer "F.Cu") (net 12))
 (segment (start 127.767 78.02) (end 127.767 90.49) (width 0.2) (layer "F.Cu") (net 12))
 (segment (start 128.757 98.746346) (end 137.16 107.188) (width 0.2) (layer "F.Cu") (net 12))
 (segment (start 176.2125 81.8005) (end 173.632 79.22) (width 0.2) (layer "F.Cu") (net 17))
 (segment (start 124.827 103.356152) (end 149.510848 128.04) (width 0.2) (layer "F.Cu") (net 17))
 (segment (start 149.510848 128.04) (end 174.331314 128.04) (width 0.2) (layer "F.Cu") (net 17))
 (segment (start 174.331314 128.04) (end 176.2125 126.158814) (width 0.2) (layer "F.Cu") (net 17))
 (segment (start 176.2125 126.158814) (end 176.2125 81.8005) (width 0.2) (layer "F.Cu") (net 17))
 (segment (start 124.827 98.27) (end 124.827 103.356152) (width 0.2) (layer "F.Cu") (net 17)))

